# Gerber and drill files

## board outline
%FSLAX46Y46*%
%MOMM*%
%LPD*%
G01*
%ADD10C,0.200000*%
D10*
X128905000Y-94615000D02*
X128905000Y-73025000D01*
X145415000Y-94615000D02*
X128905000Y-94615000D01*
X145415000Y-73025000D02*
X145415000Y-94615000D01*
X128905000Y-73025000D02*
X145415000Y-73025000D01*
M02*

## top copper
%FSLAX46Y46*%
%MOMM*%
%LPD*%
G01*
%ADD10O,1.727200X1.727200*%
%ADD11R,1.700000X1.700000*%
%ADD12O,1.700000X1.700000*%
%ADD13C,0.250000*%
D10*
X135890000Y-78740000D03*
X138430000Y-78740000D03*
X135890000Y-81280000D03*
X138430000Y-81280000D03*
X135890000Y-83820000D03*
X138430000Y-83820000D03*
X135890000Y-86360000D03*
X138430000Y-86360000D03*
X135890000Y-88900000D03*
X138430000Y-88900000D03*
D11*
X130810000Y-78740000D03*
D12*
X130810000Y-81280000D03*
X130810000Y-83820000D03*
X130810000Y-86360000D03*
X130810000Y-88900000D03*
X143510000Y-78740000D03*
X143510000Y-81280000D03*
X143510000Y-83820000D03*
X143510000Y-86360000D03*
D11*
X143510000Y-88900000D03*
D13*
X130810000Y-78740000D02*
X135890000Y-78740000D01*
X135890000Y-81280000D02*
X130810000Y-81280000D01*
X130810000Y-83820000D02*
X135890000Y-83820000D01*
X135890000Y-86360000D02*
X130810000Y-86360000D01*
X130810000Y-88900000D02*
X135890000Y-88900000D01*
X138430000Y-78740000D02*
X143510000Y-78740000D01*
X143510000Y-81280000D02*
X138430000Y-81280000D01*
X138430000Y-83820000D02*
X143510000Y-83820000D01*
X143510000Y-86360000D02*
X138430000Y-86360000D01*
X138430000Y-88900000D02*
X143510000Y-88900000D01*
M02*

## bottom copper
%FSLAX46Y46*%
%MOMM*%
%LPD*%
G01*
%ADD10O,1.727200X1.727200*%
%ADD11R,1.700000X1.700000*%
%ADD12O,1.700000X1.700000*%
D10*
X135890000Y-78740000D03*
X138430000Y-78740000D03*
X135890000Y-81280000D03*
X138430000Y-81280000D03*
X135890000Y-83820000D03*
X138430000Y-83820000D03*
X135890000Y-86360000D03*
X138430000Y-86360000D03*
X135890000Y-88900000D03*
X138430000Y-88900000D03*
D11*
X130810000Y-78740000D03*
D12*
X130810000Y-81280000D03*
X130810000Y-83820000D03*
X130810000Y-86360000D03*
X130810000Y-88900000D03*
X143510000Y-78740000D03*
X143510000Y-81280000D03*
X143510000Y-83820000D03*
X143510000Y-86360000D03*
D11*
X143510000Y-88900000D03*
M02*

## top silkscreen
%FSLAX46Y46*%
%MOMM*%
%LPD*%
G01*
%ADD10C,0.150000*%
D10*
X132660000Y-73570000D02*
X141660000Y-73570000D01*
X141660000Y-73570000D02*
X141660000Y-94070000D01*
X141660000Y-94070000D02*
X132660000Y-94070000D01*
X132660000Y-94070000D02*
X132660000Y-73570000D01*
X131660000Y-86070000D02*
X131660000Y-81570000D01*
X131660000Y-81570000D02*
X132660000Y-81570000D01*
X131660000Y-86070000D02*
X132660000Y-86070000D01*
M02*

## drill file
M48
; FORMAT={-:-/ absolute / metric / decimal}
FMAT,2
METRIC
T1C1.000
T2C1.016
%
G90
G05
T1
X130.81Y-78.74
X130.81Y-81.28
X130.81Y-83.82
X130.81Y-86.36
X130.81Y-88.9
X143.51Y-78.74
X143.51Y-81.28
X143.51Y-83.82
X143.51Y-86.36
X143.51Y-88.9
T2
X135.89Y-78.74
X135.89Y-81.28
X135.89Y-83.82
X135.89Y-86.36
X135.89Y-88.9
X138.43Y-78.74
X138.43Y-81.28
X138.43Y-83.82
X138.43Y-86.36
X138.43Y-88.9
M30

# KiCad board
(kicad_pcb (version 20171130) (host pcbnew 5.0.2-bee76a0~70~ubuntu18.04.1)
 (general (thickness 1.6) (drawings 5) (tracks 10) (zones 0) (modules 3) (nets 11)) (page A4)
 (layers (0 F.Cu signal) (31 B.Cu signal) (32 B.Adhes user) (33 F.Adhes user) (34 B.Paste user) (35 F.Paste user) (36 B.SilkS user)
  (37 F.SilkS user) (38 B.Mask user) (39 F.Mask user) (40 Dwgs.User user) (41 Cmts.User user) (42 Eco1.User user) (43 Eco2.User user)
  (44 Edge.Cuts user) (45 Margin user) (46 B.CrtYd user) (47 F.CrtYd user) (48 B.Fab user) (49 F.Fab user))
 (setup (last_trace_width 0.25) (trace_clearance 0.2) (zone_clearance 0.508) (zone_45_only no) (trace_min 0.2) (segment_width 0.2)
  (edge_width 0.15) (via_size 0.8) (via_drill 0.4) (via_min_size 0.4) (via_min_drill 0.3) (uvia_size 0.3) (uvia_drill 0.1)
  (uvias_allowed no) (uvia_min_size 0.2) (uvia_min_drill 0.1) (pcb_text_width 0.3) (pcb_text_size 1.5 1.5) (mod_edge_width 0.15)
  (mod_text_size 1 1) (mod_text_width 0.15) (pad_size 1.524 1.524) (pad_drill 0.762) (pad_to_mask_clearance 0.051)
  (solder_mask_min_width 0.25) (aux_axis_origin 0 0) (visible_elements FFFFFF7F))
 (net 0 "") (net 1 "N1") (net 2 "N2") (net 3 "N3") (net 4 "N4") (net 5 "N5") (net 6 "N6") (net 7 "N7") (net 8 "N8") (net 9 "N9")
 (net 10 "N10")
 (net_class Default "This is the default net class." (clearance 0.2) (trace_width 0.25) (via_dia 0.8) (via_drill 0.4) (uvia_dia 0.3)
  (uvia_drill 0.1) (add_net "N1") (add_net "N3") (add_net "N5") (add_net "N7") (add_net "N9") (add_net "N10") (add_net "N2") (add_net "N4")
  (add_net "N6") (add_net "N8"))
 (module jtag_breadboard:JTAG (layer F.Cu) (at 137.16 83.82)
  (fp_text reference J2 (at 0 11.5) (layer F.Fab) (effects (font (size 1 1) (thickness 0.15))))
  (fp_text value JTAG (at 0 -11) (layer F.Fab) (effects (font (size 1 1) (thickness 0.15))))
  (fp_line (start -4.5 -10.25) (end 4.5 -10.25) (layer F.SilkS) (width 0.15))
  (fp_line (start 4.5 -10.25) (end 4.5 10.25) (layer F.SilkS) (width 0.15))
  (fp_line (start 4.5 10.25) (end -4.5 10.25) (layer F.SilkS) (width 0.15))
  (fp_line (start -4.5 10.25) (end -4.5 -10.25) (layer F.SilkS) (width 0.15))
  (fp_line (start -5.5 2.25) (end -5.5 -2.25) (layer F.SilkS) (width 0.15))
  (fp_line (start -5.5 -2.25) (end -4.5 -2.25) (layer F.SilkS) (width 0.15))
  (fp_line (start -5.5 2.25) (end -4.5 2.25) (layer F.SilkS) (width 0.15))
  (pad 1 thru_hole oval (at -1.27 -5.08) (size 1.7272 1.7272) (drill 1.016) (layers *.Cu *.Mask) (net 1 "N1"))
  (pad 2 thru_hole oval (at 1.27 -5.08) (size 1.7272 1.7272) (drill 1.016) (layers *.Cu *.Mask) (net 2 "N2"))
  (pad 3 thru_hole oval (at -1.27 -2.54) (size 1.7272 1.7272) (drill 1.016) (layers *.Cu *.Mask) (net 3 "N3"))
  (pad 4 thru_hole oval (at 1.27 -2.54) (size 1.7272 1.7272) (drill 1.016) (layers *.Cu *.Mask) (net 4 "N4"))
  (pad 5 thru_hole oval (at -1.27 0) (size 1.7272 1.7272) (drill 1.016) (layers *.Cu *.Mask) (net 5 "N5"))
  (pad 6 thru_hole oval (at 1.27 0) (size 1.7272 1.7272) (drill 1.016) (layers *.Cu *.Mask) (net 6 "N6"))
  (pad 7 thru_hole oval (at -1.27 2.54) (size 1.7272 1.7272) (drill 1.016) (layers *.Cu *.Mask) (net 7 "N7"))
  (pad 8 thru_hole oval (at 1.27 2.54) (size 1.7272 1.7272) (drill 1.016) (layers *.Cu *.Mask) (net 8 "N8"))
  (pad 9 thru_hole oval (at -1.27 5.08) (size 1.7272 1.7272) (drill 1.016) (layers *.Cu *.Mask) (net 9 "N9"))
  (pad 10 thru_hole oval (at 1.27 5.08) (size 1.7272 1.7272) (drill 1.016) (layers *.Cu *.Mask) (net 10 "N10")))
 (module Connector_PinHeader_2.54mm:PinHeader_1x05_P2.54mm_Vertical (layer B.Cu) (at 130.81 78.74 180)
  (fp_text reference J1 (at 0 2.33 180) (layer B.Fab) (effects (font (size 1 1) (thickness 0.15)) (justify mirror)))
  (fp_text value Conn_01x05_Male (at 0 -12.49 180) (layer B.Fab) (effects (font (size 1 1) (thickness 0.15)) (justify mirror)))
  (pad 1 thru_hole rect (at 0 0 180) (size 1.7 1.7) (drill 1) (layers *.Cu *.Mask) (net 1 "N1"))
  (pad 2 thru_hole oval (at 0 -2.54 180) (size 1.7 1.7) (drill 1) (layers *.Cu *.Mask) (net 3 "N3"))
  (pad 3 thru_hole oval (at 0 -5.08 180) (size 1.7 1.7) (drill 1) (layers *.Cu *.Mask) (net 5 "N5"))
  (pad 4 thru_hole oval (at 0 -7.62 180) (size 1.7 1.7) (drill 1) (layers *.Cu *.Mask) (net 7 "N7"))
  (pad 5 thru_hole oval (at 0 -10.16 180) (size 1.7 1.7) (drill 1) (layers *.Cu *.Mask) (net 9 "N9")))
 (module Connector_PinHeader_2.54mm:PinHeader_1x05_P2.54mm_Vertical (layer B.Cu) (at 143.51 88.9)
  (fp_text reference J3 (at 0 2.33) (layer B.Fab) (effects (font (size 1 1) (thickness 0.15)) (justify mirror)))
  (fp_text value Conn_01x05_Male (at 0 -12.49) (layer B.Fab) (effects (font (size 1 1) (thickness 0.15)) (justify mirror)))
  (pad 5 thru_hole oval (at 0 -10.16) (size 1.7 1.7) (drill 1) (layers *.Cu *.Mask) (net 2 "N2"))
  (pad 4 thru_hole oval (at 0 -7.62) (size 1.7 1.7) (drill 1) (layers *.Cu *.Mask) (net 4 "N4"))
  (pad 3 thru_hole oval (at 0 -5.08) (size 1.7 1.7) (drill 1) (layers *.Cu *.Mask) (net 6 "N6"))
  (pad 2 thru_hole oval (at 0 -2.54) (size 1.7 1.7) (drill 1) (layers *.Cu *.Mask) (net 8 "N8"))
  (pad 1 thru_hole rect (at 0 0) (size 1.7 1.7) (drill 1) (layers *.Cu *.Mask) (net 10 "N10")))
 (gr_line (start 128.905 94.615) (end 128.905 73.025) (layer Edge.Cuts) (width 0.2))
 (gr_line (start 145.415 94.615) (end 128.905 94.615) (layer Edge.Cuts) (width 0.2))
 (gr_line (start 145.415 73.025) (end 145.415 94.615) (layer Edge.Cuts) (width 0.2))
 (gr_line (start 128.905 73.025) (end 145.415 73.025) (layer Edge.Cuts) (width 0.2))
 (segment (start 130.81 78.74) (end 135.89 78.74) (width 0.25) (layer F.Cu) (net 1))
 (segment (start 135.89 81.28) (end 130.81 81.28) (width 0.25) (layer F.Cu) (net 3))
 (segment (start 130.81 83.82) (end 135.89 83.82) (width 0.25) (layer F.Cu) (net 5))
 (segment (start 135.89 86.36) (end 130.81 86.36) (width 0.25) (layer F.Cu) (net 7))
 (segment (start 130.81 88.9) (end 135.89 88.9) (width 0.25) (layer F.Cu) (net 9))
 (segment (start 138.43 78.74) (end 143.51 78.74) (width 0.25) (layer F.Cu) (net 2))
 (segment (start 143.51 81.28) (end 138.43 81.28) (width 0.25) (layer F.Cu) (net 4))
 (segment (start 138.43 83.82) (end 143.51 83.82) (width 0.25) (layer F.Cu) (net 6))
 (segment (start 143.51 86.36) (end 138.43 86.36) (width 0.25) (layer F.Cu) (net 8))
 (segment (start 138.43 88.9) (end 143.51 88.9) (width 0.25) (layer F.Cu) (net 10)))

